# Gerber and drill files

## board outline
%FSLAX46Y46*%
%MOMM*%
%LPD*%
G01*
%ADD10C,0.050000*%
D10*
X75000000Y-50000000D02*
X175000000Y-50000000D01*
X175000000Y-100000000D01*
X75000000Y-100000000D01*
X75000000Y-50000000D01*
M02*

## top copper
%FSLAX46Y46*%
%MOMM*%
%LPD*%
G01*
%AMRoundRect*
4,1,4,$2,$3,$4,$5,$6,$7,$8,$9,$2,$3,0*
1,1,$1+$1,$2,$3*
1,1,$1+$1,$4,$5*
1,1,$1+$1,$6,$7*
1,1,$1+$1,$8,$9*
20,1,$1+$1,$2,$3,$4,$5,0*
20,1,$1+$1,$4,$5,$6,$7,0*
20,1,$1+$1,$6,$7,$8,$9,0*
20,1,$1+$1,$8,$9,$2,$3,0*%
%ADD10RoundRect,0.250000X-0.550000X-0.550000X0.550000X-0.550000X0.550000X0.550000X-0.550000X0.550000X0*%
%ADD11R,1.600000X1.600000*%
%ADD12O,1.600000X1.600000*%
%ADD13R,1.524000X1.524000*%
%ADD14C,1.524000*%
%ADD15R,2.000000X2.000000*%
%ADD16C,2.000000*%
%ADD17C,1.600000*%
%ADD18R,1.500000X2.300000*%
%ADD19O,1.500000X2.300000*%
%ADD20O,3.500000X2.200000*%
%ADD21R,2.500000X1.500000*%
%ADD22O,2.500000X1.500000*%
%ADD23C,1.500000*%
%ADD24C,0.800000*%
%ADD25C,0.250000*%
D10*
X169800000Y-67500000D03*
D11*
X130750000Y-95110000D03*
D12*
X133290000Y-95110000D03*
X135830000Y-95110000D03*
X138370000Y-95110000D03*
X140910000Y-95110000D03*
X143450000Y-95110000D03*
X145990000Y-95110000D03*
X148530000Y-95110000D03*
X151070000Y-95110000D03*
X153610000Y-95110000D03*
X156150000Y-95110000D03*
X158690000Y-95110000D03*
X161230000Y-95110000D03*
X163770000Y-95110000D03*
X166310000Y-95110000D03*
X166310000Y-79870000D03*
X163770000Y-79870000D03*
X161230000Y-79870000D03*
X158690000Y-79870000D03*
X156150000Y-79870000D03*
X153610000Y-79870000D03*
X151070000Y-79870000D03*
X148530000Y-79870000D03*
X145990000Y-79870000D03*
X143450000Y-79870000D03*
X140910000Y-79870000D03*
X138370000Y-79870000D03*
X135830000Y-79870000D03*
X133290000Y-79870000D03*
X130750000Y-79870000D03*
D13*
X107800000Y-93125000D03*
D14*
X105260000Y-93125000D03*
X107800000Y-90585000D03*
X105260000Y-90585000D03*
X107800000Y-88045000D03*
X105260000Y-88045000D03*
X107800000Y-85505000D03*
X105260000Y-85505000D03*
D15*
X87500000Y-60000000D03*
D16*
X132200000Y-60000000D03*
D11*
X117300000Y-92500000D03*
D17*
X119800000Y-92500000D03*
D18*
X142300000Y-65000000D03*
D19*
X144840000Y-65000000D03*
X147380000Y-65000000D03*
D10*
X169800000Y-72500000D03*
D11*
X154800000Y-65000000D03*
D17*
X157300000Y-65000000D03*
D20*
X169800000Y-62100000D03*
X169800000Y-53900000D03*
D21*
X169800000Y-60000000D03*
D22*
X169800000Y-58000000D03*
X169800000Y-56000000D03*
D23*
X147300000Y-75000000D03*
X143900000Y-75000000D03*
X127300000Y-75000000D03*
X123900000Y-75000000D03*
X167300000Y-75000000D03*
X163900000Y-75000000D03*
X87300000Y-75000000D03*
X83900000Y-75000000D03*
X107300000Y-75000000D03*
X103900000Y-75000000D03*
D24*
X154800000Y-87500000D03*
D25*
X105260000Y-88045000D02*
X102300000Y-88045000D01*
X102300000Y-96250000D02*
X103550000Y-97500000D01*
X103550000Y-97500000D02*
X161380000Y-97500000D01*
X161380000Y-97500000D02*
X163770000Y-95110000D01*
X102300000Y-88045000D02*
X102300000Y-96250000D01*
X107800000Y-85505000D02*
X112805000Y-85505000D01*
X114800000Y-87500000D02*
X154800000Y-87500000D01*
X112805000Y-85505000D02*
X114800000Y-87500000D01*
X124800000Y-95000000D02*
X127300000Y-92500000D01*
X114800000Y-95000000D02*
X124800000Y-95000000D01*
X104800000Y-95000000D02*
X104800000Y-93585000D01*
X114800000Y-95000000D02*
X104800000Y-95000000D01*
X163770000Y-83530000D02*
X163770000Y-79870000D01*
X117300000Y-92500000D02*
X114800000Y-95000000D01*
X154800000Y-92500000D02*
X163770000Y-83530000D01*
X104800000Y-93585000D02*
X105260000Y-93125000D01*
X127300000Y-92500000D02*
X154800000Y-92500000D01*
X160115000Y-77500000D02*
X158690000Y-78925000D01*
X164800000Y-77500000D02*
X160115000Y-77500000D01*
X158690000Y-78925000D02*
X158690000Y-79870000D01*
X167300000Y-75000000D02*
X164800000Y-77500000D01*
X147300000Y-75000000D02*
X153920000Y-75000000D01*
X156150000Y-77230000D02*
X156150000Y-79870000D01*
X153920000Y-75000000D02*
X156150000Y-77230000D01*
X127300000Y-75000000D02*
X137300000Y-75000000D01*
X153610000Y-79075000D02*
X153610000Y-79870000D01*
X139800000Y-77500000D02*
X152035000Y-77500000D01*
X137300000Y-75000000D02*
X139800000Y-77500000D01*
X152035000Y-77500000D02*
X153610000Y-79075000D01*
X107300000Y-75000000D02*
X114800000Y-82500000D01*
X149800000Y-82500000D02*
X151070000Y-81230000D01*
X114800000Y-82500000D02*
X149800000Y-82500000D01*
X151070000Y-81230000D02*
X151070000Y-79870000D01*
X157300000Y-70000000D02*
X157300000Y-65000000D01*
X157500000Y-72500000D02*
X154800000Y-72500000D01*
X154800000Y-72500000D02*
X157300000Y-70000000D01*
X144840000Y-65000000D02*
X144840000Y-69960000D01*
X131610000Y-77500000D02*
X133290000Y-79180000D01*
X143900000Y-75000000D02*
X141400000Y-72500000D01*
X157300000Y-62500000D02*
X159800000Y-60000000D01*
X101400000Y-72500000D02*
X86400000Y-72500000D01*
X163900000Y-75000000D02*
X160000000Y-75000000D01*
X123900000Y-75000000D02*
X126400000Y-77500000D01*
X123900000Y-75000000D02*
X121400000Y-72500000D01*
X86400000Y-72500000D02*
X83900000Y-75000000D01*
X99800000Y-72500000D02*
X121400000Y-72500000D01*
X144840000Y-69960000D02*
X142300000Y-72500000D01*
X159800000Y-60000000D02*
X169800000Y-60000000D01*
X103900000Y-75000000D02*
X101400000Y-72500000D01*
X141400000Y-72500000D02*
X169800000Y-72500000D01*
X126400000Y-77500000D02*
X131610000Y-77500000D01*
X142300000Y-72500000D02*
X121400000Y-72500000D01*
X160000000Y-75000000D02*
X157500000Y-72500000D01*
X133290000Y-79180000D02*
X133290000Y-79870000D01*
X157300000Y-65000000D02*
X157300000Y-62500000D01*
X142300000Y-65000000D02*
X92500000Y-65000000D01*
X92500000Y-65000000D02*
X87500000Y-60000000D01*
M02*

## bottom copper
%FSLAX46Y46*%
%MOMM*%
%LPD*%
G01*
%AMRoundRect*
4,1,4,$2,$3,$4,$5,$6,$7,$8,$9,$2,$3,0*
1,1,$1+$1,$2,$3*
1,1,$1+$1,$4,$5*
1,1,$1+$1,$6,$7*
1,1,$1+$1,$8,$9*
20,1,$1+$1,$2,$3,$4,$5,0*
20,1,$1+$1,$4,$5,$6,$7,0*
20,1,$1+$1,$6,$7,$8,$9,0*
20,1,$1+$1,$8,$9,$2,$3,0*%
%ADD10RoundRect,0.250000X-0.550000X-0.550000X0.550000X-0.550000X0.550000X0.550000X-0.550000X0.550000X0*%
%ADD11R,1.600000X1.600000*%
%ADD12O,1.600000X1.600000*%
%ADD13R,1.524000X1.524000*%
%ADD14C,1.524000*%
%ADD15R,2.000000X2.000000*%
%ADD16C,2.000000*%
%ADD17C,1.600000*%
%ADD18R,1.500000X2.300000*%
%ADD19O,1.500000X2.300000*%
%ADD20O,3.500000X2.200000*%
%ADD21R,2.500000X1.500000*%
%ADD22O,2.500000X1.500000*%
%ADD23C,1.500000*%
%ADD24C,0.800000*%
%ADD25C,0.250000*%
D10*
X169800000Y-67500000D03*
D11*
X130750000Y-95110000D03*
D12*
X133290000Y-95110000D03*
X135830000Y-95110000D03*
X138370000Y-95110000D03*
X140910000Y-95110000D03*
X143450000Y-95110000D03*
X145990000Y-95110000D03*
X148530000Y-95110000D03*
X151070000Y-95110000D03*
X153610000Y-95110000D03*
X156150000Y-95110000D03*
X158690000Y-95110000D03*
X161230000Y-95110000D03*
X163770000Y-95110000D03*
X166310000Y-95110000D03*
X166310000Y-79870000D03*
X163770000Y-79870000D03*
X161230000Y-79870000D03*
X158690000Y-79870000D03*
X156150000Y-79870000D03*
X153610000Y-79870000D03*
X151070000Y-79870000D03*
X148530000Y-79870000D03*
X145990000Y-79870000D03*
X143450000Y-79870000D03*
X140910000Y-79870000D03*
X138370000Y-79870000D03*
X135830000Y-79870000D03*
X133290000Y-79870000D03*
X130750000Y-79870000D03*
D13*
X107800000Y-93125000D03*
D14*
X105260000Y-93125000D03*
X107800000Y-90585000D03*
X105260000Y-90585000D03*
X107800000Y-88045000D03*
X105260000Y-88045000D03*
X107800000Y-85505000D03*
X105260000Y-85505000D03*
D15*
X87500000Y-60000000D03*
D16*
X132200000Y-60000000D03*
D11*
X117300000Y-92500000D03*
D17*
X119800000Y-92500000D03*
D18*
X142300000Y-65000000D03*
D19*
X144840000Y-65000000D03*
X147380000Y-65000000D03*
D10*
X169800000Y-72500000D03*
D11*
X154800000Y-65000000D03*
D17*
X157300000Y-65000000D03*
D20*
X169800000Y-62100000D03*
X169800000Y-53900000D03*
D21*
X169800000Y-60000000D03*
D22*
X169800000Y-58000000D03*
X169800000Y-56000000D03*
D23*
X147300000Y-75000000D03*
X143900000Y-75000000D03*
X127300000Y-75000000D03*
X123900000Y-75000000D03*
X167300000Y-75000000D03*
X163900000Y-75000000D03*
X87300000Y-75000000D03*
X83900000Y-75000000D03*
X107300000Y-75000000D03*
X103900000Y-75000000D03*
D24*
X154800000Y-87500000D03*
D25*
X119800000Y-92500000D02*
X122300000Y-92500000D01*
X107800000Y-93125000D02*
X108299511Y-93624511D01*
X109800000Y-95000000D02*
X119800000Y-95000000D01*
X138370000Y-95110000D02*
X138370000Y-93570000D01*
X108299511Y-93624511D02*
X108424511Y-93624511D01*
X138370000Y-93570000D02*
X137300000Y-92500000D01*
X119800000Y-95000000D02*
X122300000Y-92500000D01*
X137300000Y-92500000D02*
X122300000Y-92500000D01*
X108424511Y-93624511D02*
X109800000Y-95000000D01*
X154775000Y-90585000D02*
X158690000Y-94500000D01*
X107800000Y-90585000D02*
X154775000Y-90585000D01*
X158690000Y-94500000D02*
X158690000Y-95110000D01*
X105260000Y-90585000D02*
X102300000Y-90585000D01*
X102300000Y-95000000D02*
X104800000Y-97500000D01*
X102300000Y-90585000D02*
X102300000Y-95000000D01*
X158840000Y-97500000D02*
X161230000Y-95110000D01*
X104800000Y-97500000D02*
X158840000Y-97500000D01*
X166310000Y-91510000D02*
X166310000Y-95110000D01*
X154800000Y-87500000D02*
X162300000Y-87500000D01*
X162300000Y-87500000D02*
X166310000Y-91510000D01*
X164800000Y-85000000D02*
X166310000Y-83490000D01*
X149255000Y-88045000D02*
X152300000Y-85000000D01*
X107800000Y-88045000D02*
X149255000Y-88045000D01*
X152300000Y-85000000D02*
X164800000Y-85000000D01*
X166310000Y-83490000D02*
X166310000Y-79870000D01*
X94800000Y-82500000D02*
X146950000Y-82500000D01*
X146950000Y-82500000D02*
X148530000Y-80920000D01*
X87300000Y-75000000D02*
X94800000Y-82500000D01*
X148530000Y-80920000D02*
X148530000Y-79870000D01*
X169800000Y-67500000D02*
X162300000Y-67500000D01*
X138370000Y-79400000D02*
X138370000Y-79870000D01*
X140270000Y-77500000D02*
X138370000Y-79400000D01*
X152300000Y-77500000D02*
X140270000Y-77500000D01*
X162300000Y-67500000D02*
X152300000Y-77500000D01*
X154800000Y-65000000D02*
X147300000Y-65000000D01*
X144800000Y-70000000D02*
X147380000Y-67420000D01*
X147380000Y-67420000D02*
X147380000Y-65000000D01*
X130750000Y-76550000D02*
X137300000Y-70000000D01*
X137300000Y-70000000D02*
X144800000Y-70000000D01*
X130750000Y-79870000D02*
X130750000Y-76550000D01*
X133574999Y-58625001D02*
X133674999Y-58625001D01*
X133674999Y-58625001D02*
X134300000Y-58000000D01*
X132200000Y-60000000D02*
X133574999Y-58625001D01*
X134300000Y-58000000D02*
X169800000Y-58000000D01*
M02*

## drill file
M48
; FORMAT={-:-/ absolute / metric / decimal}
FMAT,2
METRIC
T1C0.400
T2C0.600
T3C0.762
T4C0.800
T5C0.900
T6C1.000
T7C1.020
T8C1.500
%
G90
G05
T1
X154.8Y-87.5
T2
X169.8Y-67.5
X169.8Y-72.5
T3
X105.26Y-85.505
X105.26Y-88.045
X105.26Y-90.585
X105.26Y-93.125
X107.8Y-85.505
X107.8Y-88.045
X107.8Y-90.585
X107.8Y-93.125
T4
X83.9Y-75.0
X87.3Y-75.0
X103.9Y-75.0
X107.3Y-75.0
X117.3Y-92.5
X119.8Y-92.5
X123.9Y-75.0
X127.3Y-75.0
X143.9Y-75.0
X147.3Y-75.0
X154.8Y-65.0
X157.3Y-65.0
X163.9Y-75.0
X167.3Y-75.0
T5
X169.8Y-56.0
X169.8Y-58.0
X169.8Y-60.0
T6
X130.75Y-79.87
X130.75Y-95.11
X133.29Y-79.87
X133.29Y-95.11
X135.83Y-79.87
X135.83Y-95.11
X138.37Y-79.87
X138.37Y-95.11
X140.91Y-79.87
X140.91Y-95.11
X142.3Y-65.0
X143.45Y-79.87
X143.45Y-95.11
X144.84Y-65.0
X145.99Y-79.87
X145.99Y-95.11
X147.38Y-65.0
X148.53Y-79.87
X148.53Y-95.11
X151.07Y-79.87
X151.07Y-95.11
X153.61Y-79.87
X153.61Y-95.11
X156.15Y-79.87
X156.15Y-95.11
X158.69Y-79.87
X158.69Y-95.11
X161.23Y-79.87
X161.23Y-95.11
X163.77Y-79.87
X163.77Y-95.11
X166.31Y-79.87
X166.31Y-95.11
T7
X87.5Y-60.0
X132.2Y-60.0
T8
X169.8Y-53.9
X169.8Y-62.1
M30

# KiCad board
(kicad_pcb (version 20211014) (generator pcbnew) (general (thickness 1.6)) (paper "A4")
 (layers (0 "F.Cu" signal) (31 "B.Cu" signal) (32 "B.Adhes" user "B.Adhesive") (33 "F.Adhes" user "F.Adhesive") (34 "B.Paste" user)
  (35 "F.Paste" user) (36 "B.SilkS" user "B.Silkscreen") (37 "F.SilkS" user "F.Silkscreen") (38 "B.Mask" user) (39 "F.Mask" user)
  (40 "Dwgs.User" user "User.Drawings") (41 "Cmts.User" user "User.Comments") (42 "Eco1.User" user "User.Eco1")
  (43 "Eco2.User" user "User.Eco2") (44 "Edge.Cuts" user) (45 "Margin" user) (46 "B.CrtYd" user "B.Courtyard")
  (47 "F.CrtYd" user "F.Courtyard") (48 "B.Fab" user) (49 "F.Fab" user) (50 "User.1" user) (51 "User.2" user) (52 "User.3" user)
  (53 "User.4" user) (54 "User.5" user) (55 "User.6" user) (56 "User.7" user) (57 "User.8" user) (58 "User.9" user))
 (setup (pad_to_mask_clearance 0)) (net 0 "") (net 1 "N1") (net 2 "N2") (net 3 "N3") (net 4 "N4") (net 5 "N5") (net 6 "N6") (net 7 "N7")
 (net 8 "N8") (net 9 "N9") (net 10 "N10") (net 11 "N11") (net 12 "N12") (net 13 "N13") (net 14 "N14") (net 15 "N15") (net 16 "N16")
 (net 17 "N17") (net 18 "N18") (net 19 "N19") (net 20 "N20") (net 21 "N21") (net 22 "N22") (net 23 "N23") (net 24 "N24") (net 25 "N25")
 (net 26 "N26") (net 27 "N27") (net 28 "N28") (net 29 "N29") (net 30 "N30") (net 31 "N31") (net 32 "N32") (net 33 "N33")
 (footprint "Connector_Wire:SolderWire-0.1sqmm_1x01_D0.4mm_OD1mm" (layer "F.Cu") (at 169.8 67.5)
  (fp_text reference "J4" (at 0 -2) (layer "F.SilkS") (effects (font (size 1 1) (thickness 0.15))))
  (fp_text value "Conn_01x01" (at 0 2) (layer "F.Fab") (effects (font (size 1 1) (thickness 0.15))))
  (pad "1" thru_hole roundrect (at 0 0) (size 1.6 1.6) (drill 0.6) (layers *.Cu *.Mask) (roundrect_rratio 0.15625) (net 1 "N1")))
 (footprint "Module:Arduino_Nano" (layer "F.Cu") (at 130.75 95.11 90)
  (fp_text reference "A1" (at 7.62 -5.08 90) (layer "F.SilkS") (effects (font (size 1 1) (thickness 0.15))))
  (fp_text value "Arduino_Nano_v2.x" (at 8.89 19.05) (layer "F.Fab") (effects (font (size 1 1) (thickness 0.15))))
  (pad "1" thru_hole rect (at 0 0 90) (size 1.6 1.6) (drill 1) (layers *.Cu *.Mask) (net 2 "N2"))
  (pad "2" thru_hole oval (at 0 2.54 90) (size 1.6 1.6) (drill 1) (layers *.Cu *.Mask) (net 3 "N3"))
  (pad "3" thru_hole oval (at 0 5.08 90) (size 1.6 1.6) (drill 1) (layers *.Cu *.Mask) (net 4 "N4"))
  (pad "4" thru_hole oval (at 0 7.62 90) (size 1.6 1.6) (drill 1) (layers *.Cu *.Mask) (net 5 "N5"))
  (pad "5" thru_hole oval (at 0 10.16 90) (size 1.6 1.6) (drill 1) (layers *.Cu *.Mask) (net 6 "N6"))
  (pad "6" thru_hole oval (at 0 12.7 90) (size 1.6 1.6) (drill 1) (layers *.Cu *.Mask) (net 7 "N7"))
  (pad "7" thru_hole oval (at 0 15.24 90) (size 1.6 1.6) (drill 1) (layers *.Cu *.Mask) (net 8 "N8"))
  (pad "8" thru_hole oval (at 0 17.78 90) (size 1.6 1.6) (drill 1) (layers *.Cu *.Mask) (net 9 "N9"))
  (pad "9" thru_hole oval (at 0 20.32 90) (size 1.6 1.6) (drill 1) (layers *.Cu *.Mask) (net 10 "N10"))
  (pad "10" thru_hole oval (at 0 22.86 90) (size 1.6 1.6) (drill 1) (layers *.Cu *.Mask) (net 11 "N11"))
  (pad "11" thru_hole oval (at 0 25.4 90) (size 1.6 1.6) (drill 1) (layers *.Cu *.Mask) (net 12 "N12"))
  (pad "12" thru_hole oval (at 0 27.94 90) (size 1.6 1.6) (drill 1) (layers *.Cu *.Mask) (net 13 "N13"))
  (pad "13" thru_hole oval (at 0 30.48 90) (size 1.6 1.6) (drill 1) (layers *.Cu *.Mask) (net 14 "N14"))
  (pad "14" thru_hole oval (at 0 33.02 90) (size 1.6 1.6) (drill 1) (layers *.Cu *.Mask) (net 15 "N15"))
  (pad "15" thru_hole oval (at 0 35.56 90) (size 1.6 1.6) (drill 1) (layers *.Cu *.Mask) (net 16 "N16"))
  (pad "16" thru_hole oval (at 15.24 35.56 90) (size 1.6 1.6) (drill 1) (layers *.Cu *.Mask) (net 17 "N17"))
  (pad "17" thru_hole oval (at 15.24 33.02 90) (size 1.6 1.6) (drill 1) (layers *.Cu *.Mask) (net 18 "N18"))
  (pad "18" thru_hole oval (at 15.24 30.48 90) (size 1.6 1.6) (drill 1) (layers *.Cu *.Mask) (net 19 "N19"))
  (pad "19" thru_hole oval (at 15.24 27.94 90) (size 1.6 1.6) (drill 1) (layers *.Cu *.Mask) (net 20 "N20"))
  (pad "20" thru_hole oval (at 15.24 25.4 90) (size 1.6 1.6) (drill 1) (layers *.Cu *.Mask) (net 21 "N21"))
  (pad "21" thru_hole oval (at 15.24 22.86 90) (size 1.6 1.6) (drill 1) (layers *.Cu *.Mask) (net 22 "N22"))
  (pad "22" thru_hole oval (at 15.24 20.32 90) (size 1.6 1.6) (drill 1) (layers *.Cu *.Mask) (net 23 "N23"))
  (pad "23" thru_hole oval (at 15.24 17.78 90) (size 1.6 1.6) (drill 1) (layers *.Cu *.Mask) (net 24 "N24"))
  (pad "24" thru_hole oval (at 15.24 15.24 90) (size 1.6 1.6) (drill 1) (layers *.Cu *.Mask) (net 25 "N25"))
  (pad "25" thru_hole oval (at 15.24 12.7 90) (size 1.6 1.6) (drill 1) (layers *.Cu *.Mask) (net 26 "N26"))
  (pad "26" thru_hole oval (at 15.24 10.16 90) (size 1.6 1.6) (drill 1) (layers *.Cu *.Mask) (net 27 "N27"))
  (pad "27" thru_hole oval (at 15.24 7.62 90) (size 1.6 1.6) (drill 1) (layers *.Cu *.Mask) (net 1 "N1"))
  (pad "28" thru_hole oval (at 15.24 5.08 90) (size 1.6 1.6) (drill 1) (layers *.Cu *.Mask) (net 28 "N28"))
  (pad "29" thru_hole oval (at 15.24 2.54 90) (size 1.6 1.6) (drill 1) (layers *.Cu *.Mask) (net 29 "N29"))
  (pad "30" thru_hole oval (at 15.24 0 90) (size 1.6 1.6) (drill 1) (layers *.Cu *.Mask) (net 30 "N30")))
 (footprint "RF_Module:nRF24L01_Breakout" (layer "F.Cu") (at 107.8 93.125 180)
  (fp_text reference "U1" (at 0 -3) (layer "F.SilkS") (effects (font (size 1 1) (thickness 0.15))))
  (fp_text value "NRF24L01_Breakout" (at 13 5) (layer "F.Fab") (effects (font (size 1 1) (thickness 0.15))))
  (pad "1" thru_hole rect (at 0 0 180) (size 1.524 1.524) (drill 0.762) (layers *.Cu *.Mask) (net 5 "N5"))
  (pad "2" thru_hole circle (at 2.54 0 180) (size 1.524 1.524) (drill 0.762) (layers *.Cu *.Mask) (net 18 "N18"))
  (pad "3" thru_hole circle (at 0 2.54 180) (size 1.524 1.524) (drill 0.762) (layers *.Cu *.Mask) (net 13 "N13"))
  (pad "4" thru_hole circle (at 2.54 2.54 180) (size 1.524 1.524) (drill 0.762) (layers *.Cu *.Mask) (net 14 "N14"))
  (pad "5" thru_hole circle (at 0 5.08 180) (size 1.524 1.524) (drill 0.762) (layers *.Cu *.Mask) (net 17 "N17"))
  (pad "6" thru_hole circle (at 2.54 5.08 180) (size 1.524 1.524) (drill 0.762) (layers *.Cu *.Mask) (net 15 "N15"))
  (pad "7" thru_hole circle (at 0 7.62 180) (size 1.524 1.524) (drill 0.762) (layers *.Cu *.Mask) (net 16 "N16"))
  (pad "8" thru_hole circle (at 2.54 7.62 180) (size 1.524 1.524) (drill 0.762) (layers *.Cu *.Mask) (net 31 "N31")))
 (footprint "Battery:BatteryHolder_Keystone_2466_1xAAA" (layer "F.Cu") (at 87.5 60)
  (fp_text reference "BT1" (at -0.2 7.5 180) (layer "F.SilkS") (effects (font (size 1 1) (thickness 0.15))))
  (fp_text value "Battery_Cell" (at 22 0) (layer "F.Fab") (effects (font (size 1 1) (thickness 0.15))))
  (pad "1" thru_hole rect (at 0 0) (size 2 2) (drill 1.02) (layers *.Cu *.Mask) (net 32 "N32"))
  (pad "2" thru_hole circle (at 44.7 0) (size 2 2) (drill 1.02) (layers *.Cu *.Mask) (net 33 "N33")))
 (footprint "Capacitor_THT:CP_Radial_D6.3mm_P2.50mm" (layer "F.Cu") (at 117.3 92.5)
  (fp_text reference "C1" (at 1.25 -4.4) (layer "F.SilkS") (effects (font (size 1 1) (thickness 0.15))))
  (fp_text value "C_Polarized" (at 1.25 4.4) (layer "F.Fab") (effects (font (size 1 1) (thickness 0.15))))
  (pad "1" thru_hole rect (at 0 0) (size 1.6 1.6) (drill 0.8) (layers *.Cu *.Mask) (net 18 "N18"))
  (pad "2" thru_hole circle (at 2.5 0) (size 1.6 1.6) (drill 0.8) (layers *.Cu *.Mask) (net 5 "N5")))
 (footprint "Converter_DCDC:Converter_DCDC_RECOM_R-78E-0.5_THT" (layer "F.Cu") (at 142.3 65)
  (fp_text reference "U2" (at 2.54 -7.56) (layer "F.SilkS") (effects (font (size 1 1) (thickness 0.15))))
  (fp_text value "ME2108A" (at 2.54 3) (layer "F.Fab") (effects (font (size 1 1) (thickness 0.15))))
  (pad "1" thru_hole rect (at 0 0) (size 1.5 2.3) (drill 1) (layers *.Cu *.Mask) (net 32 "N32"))
  (pad "2" thru_hole oval (at 2.54 0) (size 1.5 2.3) (drill 1) (layers *.Cu *.Mask) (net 29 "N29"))
  (pad "3" thru_hole oval (at 5.08 0) (size 1.5 2.3) (drill 1) (layers *.Cu *.Mask) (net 30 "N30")))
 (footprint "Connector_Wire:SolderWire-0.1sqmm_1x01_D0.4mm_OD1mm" (layer "F.Cu") (at 169.8 72.5)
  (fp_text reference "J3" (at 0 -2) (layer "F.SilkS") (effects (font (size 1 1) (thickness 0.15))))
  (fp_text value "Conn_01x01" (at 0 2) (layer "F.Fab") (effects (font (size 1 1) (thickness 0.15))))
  (pad "1" thru_hole roundrect (at 0 0) (size 1.6 1.6) (drill 0.6) (layers *.Cu *.Mask) (roundrect_rratio 0.15625) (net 29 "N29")))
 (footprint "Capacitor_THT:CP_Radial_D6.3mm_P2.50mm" (layer "F.Cu") (at 154.8 65)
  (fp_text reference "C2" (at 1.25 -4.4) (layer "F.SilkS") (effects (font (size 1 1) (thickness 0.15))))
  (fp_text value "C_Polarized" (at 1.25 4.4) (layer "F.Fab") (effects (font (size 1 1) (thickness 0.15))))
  (pad "1" thru_hole rect (at 0 0) (size 1.6 1.6) (drill 0.8) (layers *.Cu *.Mask) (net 30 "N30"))
  (pad "2" thru_hole circle (at 2.5 0) (size 1.6 1.6) (drill 0.8) (layers *.Cu *.Mask) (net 29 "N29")))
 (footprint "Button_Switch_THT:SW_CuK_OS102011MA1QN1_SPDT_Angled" (layer "F.Cu") (at 169.8 60 90)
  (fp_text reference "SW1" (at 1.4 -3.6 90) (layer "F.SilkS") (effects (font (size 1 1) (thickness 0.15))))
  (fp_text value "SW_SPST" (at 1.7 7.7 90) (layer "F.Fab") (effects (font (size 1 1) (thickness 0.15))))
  (pad "" thru_hole oval (at -2.1 0 90) (size 2.2 3.5) (drill 1.5) (layers *.Cu *.Mask))
  (pad "" thru_hole oval (at 6.1 0 90) (size 2.2 3.5) (drill 1.5) (layers *.Cu *.Mask))
  (pad "1" thru_hole rect (at 0 0 90) (size 1.5 2.5) (drill 0.9) (layers *.Cu *.Mask) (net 29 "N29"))
  (pad "2" thru_hole oval (at 2 0 90) (size 1.5 2.5) (drill 0.9) (layers *.Cu *.Mask) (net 33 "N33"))
  (pad "3" thru_hole oval (at 4 0 90) (size 1.5 2.5) (drill 0.9) (layers *.Cu *.Mask)))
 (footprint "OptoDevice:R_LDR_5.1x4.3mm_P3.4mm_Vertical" (layer "B.Cu") (at 147.3 75 180)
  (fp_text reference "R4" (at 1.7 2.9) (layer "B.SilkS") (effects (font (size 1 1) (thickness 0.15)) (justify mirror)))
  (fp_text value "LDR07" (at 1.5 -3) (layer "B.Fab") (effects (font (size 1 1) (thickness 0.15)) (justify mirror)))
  (pad "1" thru_hole circle (at 0 0 180) (size 1.5 1.5) (drill 0.8) (layers *.Cu *.Mask) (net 21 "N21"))
  (pad "2" thru_hole circle (at 3.4 0 180) (size 1.5 1.5) (drill 0.8) (layers *.Cu *.Mask) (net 29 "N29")))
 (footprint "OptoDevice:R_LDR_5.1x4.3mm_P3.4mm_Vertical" (layer "B.Cu") (at 127.3 75 180)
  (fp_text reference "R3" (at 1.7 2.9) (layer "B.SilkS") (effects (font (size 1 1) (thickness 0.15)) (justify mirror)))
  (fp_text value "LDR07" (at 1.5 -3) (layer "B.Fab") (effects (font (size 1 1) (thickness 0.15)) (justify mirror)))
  (pad "1" thru_hole circle (at 0 0 180) (size 1.5 1.5) (drill 0.8) (layers *.Cu *.Mask) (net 22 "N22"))
  (pad "2" thru_hole circle (at 3.4 0 180) (size 1.5 1.5) (drill 0.8) (layers *.Cu *.Mask) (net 29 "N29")))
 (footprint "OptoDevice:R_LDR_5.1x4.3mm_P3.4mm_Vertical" (layer "B.Cu") (at 167.3 75 180)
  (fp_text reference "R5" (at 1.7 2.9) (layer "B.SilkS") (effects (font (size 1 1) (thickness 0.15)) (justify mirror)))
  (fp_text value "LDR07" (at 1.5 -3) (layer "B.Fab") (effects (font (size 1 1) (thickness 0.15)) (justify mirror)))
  (pad "1" thru_hole circle (at 0 0 180) (size 1.5 1.5) (drill 0.8) (layers *.Cu *.Mask) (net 20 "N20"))
  (pad "2" thru_hole circle (at 3.4 0 180) (size 1.5 1.5) (drill 0.8) (layers *.Cu *.Mask) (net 29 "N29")))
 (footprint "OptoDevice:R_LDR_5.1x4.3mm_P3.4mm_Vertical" (layer "B.Cu") (at 87.3 75 180)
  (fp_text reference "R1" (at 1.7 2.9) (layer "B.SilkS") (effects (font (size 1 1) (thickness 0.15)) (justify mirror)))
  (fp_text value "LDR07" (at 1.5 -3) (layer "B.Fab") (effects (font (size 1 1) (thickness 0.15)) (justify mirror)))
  (pad "1" thru_hole circle (at 0 0 180) (size 1.5 1.5) (drill 0.8) (layers *.Cu *.Mask) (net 24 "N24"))
  (pad "2" thru_hole circle (at 3.4 0 180) (size 1.5 1.5) (drill 0.8) (layers *.Cu *.Mask) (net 29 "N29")))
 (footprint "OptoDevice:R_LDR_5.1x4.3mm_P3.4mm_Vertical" (layer "B.Cu") (at 107.3 75 180)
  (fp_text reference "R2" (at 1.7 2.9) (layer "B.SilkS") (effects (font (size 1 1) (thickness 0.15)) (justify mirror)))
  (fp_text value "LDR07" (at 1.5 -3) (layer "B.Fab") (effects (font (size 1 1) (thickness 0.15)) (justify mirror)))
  (pad "1" thru_hole circle (at 0 0 180) (size 1.5 1.5) (drill 0.8) (layers *.Cu *.Mask) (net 23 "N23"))
  (pad "2" thru_hole circle (at 3.4 0 180) (size 1.5 1.5) (drill 0.8) (layers *.Cu *.Mask) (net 29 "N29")))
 (gr_rect (start 75 50) (end 175 100) (layer "Edge.Cuts") (width 0.05) (fill none))
 (segment (start 119.8 92.5) (end 122.3 92.5) (width 0.25) (layer "B.Cu") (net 5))
 (segment (start 107.8 93.125) (end 108.299511 93.624511) (width 0.25) (layer "B.Cu") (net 5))
 (segment (start 109.8 95) (end 119.8 95) (width 0.25) (layer "B.Cu") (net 5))
 (segment (start 138.37 95.11) (end 138.37 93.57) (width 0.25) (layer "B.Cu") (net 5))
 (segment (start 108.299511 93.624511) (end 108.424511 93.624511) (width 0.25) (layer "B.Cu") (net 5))
 (segment (start 138.37 93.57) (end 137.3 92.5) (width 0.25) (layer "B.Cu") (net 5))
 (segment (start 119.8 95) (end 122.3 92.5) (width 0.25) (layer "B.Cu") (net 5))
 (segment (start 137.3 92.5) (end 122.3 92.5) (width 0.25) (layer "B.Cu") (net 5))
 (segment (start 108.424511 93.624511) (end 109.8 95) (width 0.25) (layer "B.Cu") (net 5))
 (segment (start 154.775 90.585) (end 158.69 94.5) (width 0.25) (layer "B.Cu") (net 13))
 (segment (start 107.8 90.585) (end 154.775 90.585) (width 0.25) (layer "B.Cu") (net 13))
 (segment (start 158.69 94.5) (end 158.69 95.11) (width 0.25) (layer "B.Cu") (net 13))
 (segment (start 105.26 90.585) (end 102.3 90.585) (width 0.25) (layer "B.Cu") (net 14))
 (segment (start 102.3 95) (end 104.8 97.5) (width 0.25) (layer "B.Cu") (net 14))
 (segment (start 102.3 90.585) (end 102.3 95) (width 0.25) (layer "B.Cu") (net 14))
 (segment (start 158.84 97.5) (end 161.23 95.11) (width 0.25) (layer "B.Cu") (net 14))
 (segment (start 104.8 97.5) (end 158.84 97.5) (width 0.25) (layer "B.Cu") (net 14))
 (segment (start 105.26 88.045) (end 102.3 88.045) (width 0.25) (layer "F.Cu") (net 15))
 (segment (start 102.3 96.25) (end 103.55 97.5) (width 0.25) (layer "F.Cu") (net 15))
 (segment (start 103.55 97.5) (end 161.38 97.5) (width 0.25) (layer "F.Cu") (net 15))
 (segment (start 161.38 97.5) (end 163.77 95.11) (width 0.25) (layer "F.Cu") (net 15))
 (segment (start 102.3 88.045) (end 102.3 96.25) (width 0.25) (layer "F.Cu") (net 15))
 (segment (start 107.8 85.505) (end 112.805 85.505) (width 0.25) (layer "F.Cu") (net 16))
 (segment (start 114.8 87.5) (end 154.8 87.5) (width 0.25) (layer "F.Cu") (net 16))
 (segment (start 112.805 85.505) (end 114.8 87.5) (width 0.25) (layer "F.Cu") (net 16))
 (via (at 154.8 87.5) (size 0.8) (drill 0.4) (layers "F.Cu" "B.Cu") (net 16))
 (segment (start 166.31 91.51) (end 166.31 95.11) (width 0.25) (layer "B.Cu") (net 16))
 (segment (start 154.8 87.5) (end 162.3 87.5) (width 0.25) (layer "B.Cu") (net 16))
 (segment (start 162.3 87.5) (end 166.31 91.51) (width 0.25) (layer "B.Cu") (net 16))
 (segment (start 164.8 85) (end 166.31 83.49) (width 0.25) (layer "B.Cu") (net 17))
 (segment (start 149.255 88.045) (end 152.3 85) (width 0.25) (layer "B.Cu") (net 17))
 (segment (start 107.8 88.045) (end 149.255 88.045) (width 0.25) (layer "B.Cu") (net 17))
 (segment (start 152.3 85) (end 164.8 85) (width 0.25) (layer "B.Cu") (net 17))
 (segment (start 166.31 83.49) (end 166.31 79.87) (width 0.25) (layer "B.Cu") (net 17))
 (segment (start 124.8 95) (end 127.3 92.5) (width 0.25) (layer "F.Cu") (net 18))
 (segment (start 114.8 95) (end 124.8 95) (width 0.25) (layer "F.Cu") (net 18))
 (segment (start 104.8 95) (end 104.8 93.585) (width 0.25) (layer "F.Cu") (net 18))
 (segment (start 114.8 95) (end 104.8 95) (width 0.25) (layer "F.Cu") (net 18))
 (segment (start 163.77 83.53) (end 163.77 79.87) (width 0.25) (layer "F.Cu") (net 18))
 (segment (start 117.3 92.5) (end 114.8 95) (width 0.25) (layer "F.Cu") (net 18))
 (segment (start 154.8 92.5) (end 163.77 83.53) (width 0.25) (layer "F.Cu") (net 18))
 (segment (start 104.8 93.585) (end 105.26 93.125) (width 0.25) (layer "F.Cu") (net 18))
 (segment (start 127.3 92.5) (end 154.8 92.5) (width 0.25) (layer "F.Cu") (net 18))
 (segment (start 160.115 77.5) (end 158.69 78.925) (width 0.25) (layer "F.Cu") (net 20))
 (segment (start 164.8 77.5) (end 160.115 77.5) (width 0.25) (layer "F.Cu") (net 20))
 (segment (start 158.69 78.925) (end 158.69 79.87) (width 0.25) (layer "F.Cu") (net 20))
 (segment (start 167.3 75) (end 164.8 77.5) (width 0.25) (layer "F.Cu") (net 20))
 (segment (start 147.3 75) (end 153.92 75) (width 0.25) (layer "F.Cu") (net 21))
 (segment (start 156.15 77.23) (end 156.15 79.87) (width 0.25) (layer "F.Cu") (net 21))
 (segment (start 153.92 75) (end 156.15 77.23) (width 0.25) (layer "F.Cu") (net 21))
 (segment (start 127.3 75) (end 137.3 75) (width 0.25) (layer "F.Cu") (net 22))
 (segment (start 153.61 79.075) (end 153.61 79.87) (width 0.25) (layer "F.Cu") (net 22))
 (segment (start 139.8 77.5) (end 152.035 77.5) (width 0.25) (layer "F.Cu") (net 22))
 (segment (start 137.3 75) (end 139.8 77.5) (width 0.25) (layer "F.Cu") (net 22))
 (segment (start 152.035 77.5) (end 153.61 79.075) (width 0.25) (layer "F.Cu") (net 22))
 (segment (start 107.3 75) (end 114.8 82.5) (width 0.25) (layer "F.Cu") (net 23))
 (segment (start 149.8 82.5) (end 151.07 81.23) (width 0.25) (layer "F.Cu") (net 23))
 (segment (start 114.8 82.5) (end 149.8 82.5) (width 0.25) (layer "F.Cu") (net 23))
 (segment (start 151.07 81.23) (end 151.07 79.87) (width 0.25) (layer "F.Cu") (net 23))
 (segment (start 94.8 82.5) (end 146.95 82.5) (width 0.25) (layer "B.Cu") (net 24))
 (segment (start 146.95 82.5) (end 148.53 80.92) (width 0.25) (layer "B.Cu") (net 24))
 (segment (start 87.3 75) (end 94.8 82.5) (width 0.25) (layer "B.Cu") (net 24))
 (segment (start 148.53 80.92) (end 148.53 79.87) (width 0.25) (layer "B.Cu") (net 24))
 (segment (start 169.8 67.5) (end 162.3 67.5) (width 0.25) (layer "B.Cu") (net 1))
 (segment (start 138.37 79.4) (end 138.37 79.87) (width 0.25) (layer "B.Cu") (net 1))
 (segment (start 140.27 77.5) (end 138.37 79.4) (width 0.25) (layer "B.Cu") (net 1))
 (segment (start 152.3 77.5) (end 140.27 77.5) (width 0.25) (layer "B.Cu") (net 1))
 (segment (start 162.3 67.5) (end 152.3 77.5) (width 0.25) (layer "B.Cu") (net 1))
 (segment (start 157.3 70) (end 157.3 65) (width 0.25) (layer "F.Cu") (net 29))
 (segment (start 157.5 72.5) (end 154.8 72.5) (width 0.25) (layer "F.Cu") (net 29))
 (segment (start 154.8 72.5) (end 157.3 70) (width 0.25) (layer "F.Cu") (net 29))
 (segment (start 144.84 65) (end 144.84 69.96) (width 0.25) (layer "F.Cu") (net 29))
 (segment (start 131.61 77.5) (end 133.29 79.18) (width 0.25) (layer "F.Cu") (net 29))
 (segment (start 143.9 75) (end 141.4 72.5) (width 0.25) (layer "F.Cu") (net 29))
 (segment (start 157.3 62.5) (end 159.8 60) (width 0.25) (layer "F.Cu") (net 29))
 (segment (start 101.4 72.5) (end 86.4 72.5) (width 0.25) (layer "F.Cu") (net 29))
 (segment (start 163.9 75) (end 160 75) (width 0.25) (layer "F.Cu") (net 29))
 (segment (start 123.9 75) (end 126.4 77.5) (width 0.25) (layer "F.Cu") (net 29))
 (segment (start 123.9 75) (end 121.4 72.5) (width 0.25) (layer "F.Cu") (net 29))
 (segment (start 86.4 72.5) (end 83.9 75) (width 0.25) (layer "F.Cu") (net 29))
 (segment (start 99.8 72.5) (end 121.4 72.5) (width 0.25) (layer "F.Cu") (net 29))
 (segment (start 144.84 69.96) (end 142.3 72.5) (width 0.25) (layer "F.Cu") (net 29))
 (segment (start 159.8 60) (end 169.8 60) (width 0.25) (layer "F.Cu") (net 29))
 (segment (start 103.9 75) (end 101.4 72.5) (width 0.25) (layer "F.Cu") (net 29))
 (segment (start 141.4 72.5) (end 169.8 72.5) (width 0.25) (layer "F.Cu") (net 29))
 (segment (start 126.4 77.5) (end 131.61 77.5) (width 0.25) (layer "F.Cu") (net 29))
 (segment (start 142.3 72.5) (end 121.4 72.5) (width 0.25) (layer "F.Cu") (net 29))
 (segment (start 160 75) (end 157.5 72.5) (width 0.25) (layer "F.Cu") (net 29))
 (segment (start 133.29 79.18) (end 133.29 79.87) (width 0.25) (layer "F.Cu") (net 29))
 (segment (start 157.3 65) (end 157.3 62.5) (width 0.25) (layer "F.Cu") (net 29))
 (segment (start 154.8 65) (end 147.3 65) (width 0.25) (layer "B.Cu") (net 30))
 (segment (start 144.8 70) (end 147.38 67.42) (width 0.25) (layer "B.Cu") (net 30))
 (segment (start 147.38 67.42) (end 147.38 65) (width 0.25) (layer "B.Cu") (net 30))
 (segment (start 130.75 76.55) (end 137.3 70) (width 0.25) (layer "B.Cu") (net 30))
 (segment (start 137.3 70) (end 144.8 70) (width 0.25) (layer "B.Cu") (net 30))
 (segment (start 130.75 79.87) (end 130.75 76.55) (width 0.25) (layer "B.Cu") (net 30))
 (segment (start 142.3 65) (end 92.5 65) (width 0.25) (layer "F.Cu") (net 32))
 (segment (start 92.5 65) (end 87.5 60) (width 0.25) (layer "F.Cu") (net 32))
 (segment (start 133.574999 58.625001) (end 133.674999 58.625001) (width 0.25) (layer "B.Cu") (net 33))
 (segment (start 133.674999 58.625001) (end 134.3 58) (width 0.25) (layer "B.Cu") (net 33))
 (segment (start 132.2 60) (end 133.574999 58.625001) (width 0.25) (layer "B.Cu") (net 33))
 (segment (start 134.3 58) (end 169.8 58) (width 0.25) (layer "B.Cu") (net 33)))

